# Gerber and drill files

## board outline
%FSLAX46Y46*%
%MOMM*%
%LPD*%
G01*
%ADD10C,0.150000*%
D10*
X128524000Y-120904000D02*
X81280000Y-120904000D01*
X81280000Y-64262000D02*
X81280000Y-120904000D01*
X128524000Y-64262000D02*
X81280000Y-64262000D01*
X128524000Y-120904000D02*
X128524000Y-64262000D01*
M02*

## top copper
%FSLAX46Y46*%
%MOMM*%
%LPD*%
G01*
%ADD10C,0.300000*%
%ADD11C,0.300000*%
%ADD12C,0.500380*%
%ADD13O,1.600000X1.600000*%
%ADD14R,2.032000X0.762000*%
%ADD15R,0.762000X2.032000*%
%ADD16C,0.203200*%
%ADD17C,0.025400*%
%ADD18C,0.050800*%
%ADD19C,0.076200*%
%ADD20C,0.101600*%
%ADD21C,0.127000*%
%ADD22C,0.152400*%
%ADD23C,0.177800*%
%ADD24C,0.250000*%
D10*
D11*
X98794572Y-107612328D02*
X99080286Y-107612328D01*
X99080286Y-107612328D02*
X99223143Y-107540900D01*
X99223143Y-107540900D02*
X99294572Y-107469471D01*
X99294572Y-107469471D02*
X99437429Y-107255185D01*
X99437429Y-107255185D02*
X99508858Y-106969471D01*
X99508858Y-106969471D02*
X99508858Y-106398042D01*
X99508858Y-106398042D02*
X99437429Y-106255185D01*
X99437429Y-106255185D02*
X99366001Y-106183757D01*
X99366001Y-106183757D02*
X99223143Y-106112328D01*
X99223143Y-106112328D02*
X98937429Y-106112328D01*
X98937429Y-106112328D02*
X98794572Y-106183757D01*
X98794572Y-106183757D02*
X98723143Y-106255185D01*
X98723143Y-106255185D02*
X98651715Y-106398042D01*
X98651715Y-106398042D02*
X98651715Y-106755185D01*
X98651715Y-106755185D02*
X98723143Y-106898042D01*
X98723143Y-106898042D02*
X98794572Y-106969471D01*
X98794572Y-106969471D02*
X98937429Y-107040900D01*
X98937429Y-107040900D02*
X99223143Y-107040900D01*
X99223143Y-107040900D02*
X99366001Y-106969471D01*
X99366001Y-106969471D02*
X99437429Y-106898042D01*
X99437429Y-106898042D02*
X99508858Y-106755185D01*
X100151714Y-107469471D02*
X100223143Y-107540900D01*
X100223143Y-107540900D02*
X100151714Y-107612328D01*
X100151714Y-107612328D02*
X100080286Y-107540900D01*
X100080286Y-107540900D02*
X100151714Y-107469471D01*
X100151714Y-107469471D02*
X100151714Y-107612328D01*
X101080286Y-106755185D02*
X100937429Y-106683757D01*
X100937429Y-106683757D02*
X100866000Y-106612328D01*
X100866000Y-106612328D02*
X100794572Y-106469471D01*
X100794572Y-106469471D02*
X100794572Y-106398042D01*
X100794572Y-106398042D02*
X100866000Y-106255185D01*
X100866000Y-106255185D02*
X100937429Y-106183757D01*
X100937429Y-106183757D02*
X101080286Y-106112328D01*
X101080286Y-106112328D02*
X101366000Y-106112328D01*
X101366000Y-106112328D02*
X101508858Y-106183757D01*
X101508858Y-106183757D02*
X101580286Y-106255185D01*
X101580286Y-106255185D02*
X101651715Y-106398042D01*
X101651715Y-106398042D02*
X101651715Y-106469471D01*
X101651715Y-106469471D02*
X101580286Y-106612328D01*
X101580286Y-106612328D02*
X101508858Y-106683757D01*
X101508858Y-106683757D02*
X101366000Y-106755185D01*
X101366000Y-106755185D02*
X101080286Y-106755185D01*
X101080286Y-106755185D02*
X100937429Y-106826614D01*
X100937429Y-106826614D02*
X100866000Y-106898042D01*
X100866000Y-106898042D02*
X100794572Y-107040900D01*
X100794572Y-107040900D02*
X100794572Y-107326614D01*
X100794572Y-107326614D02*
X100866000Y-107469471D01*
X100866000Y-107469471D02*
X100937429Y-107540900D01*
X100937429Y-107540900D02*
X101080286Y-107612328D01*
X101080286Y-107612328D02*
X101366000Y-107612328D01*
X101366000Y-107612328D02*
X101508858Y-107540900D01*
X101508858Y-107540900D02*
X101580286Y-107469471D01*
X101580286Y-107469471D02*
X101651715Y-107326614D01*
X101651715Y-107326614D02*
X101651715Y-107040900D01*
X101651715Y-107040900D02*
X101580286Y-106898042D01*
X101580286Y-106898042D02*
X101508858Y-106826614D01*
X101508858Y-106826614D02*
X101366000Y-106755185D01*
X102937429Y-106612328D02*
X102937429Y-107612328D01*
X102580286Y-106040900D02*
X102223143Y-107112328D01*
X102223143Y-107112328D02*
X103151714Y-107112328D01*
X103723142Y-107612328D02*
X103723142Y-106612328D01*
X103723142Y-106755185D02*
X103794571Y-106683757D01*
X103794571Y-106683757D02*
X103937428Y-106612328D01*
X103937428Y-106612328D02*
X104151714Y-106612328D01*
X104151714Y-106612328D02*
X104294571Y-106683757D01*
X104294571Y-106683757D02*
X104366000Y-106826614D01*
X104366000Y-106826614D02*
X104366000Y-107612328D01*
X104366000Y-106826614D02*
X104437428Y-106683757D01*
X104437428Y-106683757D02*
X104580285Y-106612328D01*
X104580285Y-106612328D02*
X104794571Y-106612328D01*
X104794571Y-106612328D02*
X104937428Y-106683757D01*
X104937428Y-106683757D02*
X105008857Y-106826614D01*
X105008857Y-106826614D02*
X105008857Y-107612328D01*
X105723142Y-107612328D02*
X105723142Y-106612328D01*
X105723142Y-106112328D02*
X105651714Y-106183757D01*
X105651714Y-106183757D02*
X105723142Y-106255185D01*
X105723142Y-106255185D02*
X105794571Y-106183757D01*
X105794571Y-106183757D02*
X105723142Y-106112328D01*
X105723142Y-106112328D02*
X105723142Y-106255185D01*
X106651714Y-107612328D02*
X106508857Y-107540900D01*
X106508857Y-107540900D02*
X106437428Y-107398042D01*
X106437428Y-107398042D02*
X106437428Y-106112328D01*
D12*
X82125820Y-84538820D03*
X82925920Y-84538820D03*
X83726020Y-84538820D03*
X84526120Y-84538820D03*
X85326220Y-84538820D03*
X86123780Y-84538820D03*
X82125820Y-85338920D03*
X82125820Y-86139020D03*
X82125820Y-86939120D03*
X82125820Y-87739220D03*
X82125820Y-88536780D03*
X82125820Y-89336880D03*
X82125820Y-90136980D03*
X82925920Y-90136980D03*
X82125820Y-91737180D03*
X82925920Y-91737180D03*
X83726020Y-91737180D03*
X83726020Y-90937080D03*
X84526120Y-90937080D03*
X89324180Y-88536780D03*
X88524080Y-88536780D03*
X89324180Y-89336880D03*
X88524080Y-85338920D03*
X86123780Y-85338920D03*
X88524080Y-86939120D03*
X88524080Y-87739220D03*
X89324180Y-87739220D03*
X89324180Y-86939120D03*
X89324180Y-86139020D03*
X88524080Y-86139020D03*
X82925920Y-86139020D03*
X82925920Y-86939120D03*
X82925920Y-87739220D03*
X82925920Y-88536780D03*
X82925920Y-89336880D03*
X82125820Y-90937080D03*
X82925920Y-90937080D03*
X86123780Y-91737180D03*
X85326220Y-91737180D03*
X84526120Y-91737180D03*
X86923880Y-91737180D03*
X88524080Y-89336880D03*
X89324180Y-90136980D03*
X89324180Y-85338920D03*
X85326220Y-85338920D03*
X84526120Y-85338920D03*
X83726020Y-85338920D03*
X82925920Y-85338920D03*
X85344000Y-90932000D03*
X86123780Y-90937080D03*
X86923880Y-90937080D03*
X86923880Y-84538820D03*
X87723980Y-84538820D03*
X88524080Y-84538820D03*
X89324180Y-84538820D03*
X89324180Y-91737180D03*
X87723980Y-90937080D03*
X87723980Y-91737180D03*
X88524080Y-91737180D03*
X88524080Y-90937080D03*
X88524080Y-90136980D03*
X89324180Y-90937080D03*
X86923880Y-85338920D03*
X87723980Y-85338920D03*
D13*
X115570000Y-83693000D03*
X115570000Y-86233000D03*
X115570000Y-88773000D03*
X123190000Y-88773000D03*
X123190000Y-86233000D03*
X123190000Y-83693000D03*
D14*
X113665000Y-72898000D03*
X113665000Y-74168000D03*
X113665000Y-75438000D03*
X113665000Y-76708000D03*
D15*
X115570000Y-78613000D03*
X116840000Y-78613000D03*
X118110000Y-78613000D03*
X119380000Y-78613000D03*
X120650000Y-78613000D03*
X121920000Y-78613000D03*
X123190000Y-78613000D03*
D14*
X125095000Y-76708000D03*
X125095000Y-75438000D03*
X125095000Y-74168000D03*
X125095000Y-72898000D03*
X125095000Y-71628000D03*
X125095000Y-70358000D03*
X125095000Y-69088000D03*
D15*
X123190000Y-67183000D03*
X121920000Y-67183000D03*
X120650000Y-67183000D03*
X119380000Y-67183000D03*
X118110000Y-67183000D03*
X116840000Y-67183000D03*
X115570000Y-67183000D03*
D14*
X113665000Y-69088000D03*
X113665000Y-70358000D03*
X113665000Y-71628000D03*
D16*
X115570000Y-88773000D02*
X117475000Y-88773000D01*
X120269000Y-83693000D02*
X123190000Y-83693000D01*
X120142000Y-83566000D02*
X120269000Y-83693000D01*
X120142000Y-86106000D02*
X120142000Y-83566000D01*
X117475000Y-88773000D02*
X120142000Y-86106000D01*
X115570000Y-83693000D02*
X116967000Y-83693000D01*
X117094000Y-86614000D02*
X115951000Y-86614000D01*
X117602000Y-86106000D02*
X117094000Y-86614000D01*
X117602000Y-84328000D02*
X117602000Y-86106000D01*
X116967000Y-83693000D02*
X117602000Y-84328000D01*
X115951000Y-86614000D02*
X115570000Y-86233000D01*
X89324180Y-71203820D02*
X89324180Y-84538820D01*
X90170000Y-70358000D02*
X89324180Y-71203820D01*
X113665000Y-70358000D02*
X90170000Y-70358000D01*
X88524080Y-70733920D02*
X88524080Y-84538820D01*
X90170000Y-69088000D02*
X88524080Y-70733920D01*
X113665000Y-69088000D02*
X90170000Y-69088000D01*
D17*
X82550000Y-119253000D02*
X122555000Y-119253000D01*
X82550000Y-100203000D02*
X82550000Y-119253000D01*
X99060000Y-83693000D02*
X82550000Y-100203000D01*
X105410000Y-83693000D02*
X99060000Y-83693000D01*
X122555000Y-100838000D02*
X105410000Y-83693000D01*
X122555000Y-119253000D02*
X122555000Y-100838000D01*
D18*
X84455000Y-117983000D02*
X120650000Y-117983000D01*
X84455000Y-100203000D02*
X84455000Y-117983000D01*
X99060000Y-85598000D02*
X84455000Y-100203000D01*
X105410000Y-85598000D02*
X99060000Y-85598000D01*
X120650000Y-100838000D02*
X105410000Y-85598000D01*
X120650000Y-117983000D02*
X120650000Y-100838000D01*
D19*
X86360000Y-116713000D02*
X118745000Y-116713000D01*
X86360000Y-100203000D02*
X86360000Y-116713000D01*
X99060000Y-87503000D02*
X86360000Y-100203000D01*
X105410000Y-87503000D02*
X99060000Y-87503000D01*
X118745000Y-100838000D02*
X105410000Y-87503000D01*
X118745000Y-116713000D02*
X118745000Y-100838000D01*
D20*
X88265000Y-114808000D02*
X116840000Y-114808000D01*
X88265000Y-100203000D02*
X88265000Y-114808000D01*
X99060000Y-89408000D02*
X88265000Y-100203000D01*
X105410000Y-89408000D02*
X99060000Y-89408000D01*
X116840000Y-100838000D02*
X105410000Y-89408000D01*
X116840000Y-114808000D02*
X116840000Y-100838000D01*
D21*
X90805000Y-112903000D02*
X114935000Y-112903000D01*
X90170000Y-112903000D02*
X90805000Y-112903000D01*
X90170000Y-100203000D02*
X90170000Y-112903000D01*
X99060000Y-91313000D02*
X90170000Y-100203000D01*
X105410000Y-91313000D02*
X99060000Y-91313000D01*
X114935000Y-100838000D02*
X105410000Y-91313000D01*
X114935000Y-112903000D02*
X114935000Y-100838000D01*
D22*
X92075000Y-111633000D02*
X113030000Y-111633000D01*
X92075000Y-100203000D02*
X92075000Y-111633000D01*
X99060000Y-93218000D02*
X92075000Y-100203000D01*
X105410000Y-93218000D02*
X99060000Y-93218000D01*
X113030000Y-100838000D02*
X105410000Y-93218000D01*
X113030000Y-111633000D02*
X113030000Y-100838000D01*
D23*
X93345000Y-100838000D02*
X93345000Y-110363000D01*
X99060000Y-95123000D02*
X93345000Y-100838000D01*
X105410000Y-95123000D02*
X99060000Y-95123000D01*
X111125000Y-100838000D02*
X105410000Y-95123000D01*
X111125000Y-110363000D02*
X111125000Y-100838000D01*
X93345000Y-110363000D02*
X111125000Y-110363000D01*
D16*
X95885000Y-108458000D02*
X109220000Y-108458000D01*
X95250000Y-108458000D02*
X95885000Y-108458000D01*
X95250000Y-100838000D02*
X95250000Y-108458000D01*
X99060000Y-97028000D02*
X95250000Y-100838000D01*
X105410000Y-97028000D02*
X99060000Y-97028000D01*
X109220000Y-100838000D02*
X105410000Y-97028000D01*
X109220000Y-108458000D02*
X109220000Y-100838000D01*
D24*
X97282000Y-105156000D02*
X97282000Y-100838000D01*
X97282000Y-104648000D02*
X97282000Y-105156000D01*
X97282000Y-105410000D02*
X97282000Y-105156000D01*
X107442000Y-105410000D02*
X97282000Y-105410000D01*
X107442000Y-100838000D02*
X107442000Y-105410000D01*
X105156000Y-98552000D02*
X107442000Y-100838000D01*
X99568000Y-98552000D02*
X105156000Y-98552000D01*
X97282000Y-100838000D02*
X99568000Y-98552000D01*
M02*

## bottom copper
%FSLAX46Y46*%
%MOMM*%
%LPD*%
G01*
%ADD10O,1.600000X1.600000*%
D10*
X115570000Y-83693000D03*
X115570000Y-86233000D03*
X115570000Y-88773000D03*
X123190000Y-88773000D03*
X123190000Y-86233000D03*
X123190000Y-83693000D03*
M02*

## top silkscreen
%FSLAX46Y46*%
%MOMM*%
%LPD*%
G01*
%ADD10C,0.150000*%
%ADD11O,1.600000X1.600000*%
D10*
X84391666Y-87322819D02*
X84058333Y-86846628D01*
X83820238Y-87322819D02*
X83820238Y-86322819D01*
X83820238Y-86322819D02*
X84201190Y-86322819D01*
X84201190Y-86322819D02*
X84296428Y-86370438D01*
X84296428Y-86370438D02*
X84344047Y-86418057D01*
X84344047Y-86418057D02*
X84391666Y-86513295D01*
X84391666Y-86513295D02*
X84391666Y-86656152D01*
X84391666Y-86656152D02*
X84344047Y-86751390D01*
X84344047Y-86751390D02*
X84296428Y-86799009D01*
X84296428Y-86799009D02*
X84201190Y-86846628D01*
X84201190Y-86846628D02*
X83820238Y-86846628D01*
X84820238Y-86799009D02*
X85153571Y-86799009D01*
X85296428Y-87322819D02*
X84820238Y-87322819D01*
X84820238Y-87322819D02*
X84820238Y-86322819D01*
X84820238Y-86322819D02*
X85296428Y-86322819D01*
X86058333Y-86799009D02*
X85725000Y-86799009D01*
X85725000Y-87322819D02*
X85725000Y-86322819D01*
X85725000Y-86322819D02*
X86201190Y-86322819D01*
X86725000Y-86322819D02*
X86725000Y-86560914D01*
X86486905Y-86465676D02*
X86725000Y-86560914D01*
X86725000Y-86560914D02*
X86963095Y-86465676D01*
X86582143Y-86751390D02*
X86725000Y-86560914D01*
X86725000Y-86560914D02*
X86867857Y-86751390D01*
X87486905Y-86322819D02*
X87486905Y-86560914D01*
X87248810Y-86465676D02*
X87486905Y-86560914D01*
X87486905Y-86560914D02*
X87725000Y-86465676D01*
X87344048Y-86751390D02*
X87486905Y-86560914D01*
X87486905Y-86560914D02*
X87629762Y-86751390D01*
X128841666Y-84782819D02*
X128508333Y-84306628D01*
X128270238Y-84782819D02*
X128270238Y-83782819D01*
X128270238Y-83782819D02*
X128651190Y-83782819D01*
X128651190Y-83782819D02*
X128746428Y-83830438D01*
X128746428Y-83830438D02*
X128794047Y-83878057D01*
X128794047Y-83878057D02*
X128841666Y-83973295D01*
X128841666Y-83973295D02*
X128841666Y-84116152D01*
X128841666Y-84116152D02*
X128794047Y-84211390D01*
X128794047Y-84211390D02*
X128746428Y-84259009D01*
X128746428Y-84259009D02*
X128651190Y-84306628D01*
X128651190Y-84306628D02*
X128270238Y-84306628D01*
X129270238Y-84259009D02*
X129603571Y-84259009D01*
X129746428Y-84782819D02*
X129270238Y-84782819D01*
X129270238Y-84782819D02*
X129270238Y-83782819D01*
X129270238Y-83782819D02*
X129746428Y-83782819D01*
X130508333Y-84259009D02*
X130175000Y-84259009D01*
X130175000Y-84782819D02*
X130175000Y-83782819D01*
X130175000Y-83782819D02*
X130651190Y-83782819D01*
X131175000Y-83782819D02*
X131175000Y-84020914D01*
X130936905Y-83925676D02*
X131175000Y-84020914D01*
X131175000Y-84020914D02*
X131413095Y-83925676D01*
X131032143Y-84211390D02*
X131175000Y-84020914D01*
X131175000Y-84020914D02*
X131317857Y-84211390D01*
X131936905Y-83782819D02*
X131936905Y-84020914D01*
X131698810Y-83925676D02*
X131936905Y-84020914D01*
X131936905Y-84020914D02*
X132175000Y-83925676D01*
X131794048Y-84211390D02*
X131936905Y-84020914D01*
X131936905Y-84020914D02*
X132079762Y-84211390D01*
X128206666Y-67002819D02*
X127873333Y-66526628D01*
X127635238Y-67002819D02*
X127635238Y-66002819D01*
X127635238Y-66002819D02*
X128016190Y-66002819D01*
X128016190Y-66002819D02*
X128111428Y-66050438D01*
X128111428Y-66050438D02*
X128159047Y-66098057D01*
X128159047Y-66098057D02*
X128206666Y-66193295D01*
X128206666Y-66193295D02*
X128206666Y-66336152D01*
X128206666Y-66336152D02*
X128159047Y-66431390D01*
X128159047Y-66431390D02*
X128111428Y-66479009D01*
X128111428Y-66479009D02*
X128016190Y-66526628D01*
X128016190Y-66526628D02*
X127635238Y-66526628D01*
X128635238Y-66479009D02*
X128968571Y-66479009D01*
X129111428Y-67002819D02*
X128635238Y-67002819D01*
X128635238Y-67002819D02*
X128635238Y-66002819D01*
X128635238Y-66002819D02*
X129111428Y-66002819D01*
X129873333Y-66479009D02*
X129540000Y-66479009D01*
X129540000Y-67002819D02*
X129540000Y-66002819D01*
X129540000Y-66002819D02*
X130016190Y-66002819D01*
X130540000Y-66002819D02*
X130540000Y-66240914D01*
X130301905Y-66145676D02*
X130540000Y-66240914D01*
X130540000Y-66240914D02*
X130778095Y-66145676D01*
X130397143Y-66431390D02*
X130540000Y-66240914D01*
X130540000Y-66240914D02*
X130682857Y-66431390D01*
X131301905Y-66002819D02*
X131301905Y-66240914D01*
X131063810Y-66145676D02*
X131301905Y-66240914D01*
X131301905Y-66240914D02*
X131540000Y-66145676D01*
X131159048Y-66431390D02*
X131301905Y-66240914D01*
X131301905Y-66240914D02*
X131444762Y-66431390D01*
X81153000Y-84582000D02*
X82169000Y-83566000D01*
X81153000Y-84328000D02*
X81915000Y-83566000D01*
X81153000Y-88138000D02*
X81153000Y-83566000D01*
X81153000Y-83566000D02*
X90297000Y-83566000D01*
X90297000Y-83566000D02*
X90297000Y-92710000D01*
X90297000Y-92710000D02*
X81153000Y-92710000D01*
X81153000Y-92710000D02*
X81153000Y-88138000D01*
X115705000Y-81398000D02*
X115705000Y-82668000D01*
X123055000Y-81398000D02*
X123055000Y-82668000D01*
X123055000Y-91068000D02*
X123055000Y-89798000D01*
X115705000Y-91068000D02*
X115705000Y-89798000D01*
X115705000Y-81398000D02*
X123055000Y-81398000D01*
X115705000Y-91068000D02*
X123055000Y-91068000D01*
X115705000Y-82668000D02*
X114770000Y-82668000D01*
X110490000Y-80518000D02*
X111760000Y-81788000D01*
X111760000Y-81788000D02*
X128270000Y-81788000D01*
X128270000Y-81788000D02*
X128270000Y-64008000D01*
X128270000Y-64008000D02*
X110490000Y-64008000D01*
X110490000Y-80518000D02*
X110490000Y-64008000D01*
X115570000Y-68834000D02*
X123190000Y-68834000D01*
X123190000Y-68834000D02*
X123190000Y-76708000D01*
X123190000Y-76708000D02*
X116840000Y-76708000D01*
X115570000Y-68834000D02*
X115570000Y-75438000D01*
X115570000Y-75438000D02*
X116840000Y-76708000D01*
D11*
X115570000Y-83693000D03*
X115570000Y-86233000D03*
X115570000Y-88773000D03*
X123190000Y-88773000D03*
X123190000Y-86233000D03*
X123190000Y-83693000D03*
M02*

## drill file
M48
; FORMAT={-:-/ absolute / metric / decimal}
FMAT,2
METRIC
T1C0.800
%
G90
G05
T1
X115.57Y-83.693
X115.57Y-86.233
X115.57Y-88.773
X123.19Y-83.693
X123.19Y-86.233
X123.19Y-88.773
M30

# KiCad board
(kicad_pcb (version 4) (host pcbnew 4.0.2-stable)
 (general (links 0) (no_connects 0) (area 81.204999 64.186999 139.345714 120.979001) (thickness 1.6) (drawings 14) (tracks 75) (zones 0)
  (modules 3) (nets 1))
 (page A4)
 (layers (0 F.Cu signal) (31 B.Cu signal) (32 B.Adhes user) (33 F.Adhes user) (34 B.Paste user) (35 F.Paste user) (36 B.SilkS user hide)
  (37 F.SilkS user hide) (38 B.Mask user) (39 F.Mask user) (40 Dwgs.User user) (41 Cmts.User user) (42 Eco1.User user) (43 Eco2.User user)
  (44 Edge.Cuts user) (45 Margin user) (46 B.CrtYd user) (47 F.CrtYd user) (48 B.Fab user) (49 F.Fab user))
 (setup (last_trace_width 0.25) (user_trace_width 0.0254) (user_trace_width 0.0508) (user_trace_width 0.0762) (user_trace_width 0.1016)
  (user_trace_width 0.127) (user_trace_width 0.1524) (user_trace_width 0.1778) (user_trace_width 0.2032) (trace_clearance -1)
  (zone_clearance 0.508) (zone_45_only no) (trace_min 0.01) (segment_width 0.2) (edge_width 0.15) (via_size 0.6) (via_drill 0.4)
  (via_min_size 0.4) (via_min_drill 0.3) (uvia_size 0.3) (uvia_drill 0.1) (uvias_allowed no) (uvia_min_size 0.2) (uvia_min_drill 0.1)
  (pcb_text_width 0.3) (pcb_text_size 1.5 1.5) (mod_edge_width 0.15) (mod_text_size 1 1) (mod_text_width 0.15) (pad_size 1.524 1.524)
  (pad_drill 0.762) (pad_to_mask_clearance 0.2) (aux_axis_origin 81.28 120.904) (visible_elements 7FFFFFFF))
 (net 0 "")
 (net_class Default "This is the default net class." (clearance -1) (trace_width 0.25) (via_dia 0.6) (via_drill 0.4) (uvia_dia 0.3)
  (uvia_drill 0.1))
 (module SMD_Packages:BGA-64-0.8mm (layer F.Cu) (at 85.725 88.138)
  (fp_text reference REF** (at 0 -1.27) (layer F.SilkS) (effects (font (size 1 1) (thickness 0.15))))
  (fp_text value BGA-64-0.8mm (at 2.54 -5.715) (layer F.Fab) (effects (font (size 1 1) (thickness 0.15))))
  (fp_line (start -4.572 -3.556) (end -3.556 -4.572) (layer F.SilkS) (width 0.15))
  (fp_line (start -4.572 -3.81) (end -3.81 -4.572) (layer F.SilkS) (width 0.15))
  (fp_line (start -4.572 0) (end -4.572 -4.572) (layer F.SilkS) (width 0.15))
  (fp_line (start -4.572 -4.572) (end 4.572 -4.572) (layer F.SilkS) (width 0.15))
  (fp_line (start 4.572 -4.572) (end 4.572 4.572) (layer F.SilkS) (width 0.15))
  (fp_line (start 4.572 4.572) (end -4.572 4.572) (layer F.SilkS) (width 0.15))
  (fp_line (start -4.572 4.572) (end -4.572 0) (layer F.SilkS) (width 0.15))
  (pad A1 smd circle (at -3.59918 -3.59918) (size 0.50038 0.50038) (layers F.Cu F.Paste F.Mask))
  (pad A2 smd circle (at -2.79908 -3.59918) (size 0.50038 0.50038) (layers F.Cu F.Paste F.Mask))
  (pad A3 smd circle (at -1.99898 -3.59918) (size 0.50038 0.50038) (layers F.Cu F.Paste F.Mask))
  (pad A4 smd circle (at -1.19888 -3.59918) (size 0.50038 0.50038) (layers F.Cu F.Paste F.Mask))
  (pad A5 smd circle (at -0.39878 -3.59918) (size 0.50038 0.50038) (layers F.Cu F.Paste F.Mask))
  (pad A6 smd circle (at 0.39878 -3.59918) (size 0.50038 0.50038) (layers F.Cu F.Paste F.Mask))
  (pad B1 smd circle (at -3.59918 -2.79908) (size 0.50038 0.50038) (layers F.Cu F.Paste F.Mask))
  (pad C1 smd circle (at -3.59918 -1.99898) (size 0.50038 0.50038) (layers F.Cu F.Paste F.Mask))
  (pad D1 smd circle (at -3.59918 -1.19888) (size 0.50038 0.50038) (layers F.Cu F.Paste F.Mask))
  (pad E1 smd circle (at -3.59918 -0.39878) (size 0.50038 0.50038) (layers F.Cu F.Paste F.Mask))
  (pad F1 smd circle (at -3.59918 0.39878) (size 0.50038 0.50038) (layers F.Cu F.Paste F.Mask))
  (pad G1 smd circle (at -3.59918 1.19888) (size 0.50038 0.50038) (layers F.Cu F.Paste F.Mask))
  (pad H1 smd circle (at -3.59918 1.99898) (size 0.50038 0.50038) (layers F.Cu F.Paste F.Mask))
  (pad H2 smd circle (at -2.79908 1.99898) (size 0.50038 0.50038) (layers F.Cu F.Paste F.Mask))
  (pad K1 smd circle (at -3.59918 3.59918) (size 0.50038 0.50038) (layers F.Cu F.Paste F.Mask))
  (pad K2 smd circle (at -2.79908 3.59918) (size 0.50038 0.50038) (layers F.Cu F.Paste F.Mask))
  (pad K3 smd circle (at -1.99898 3.59918) (size 0.50038 0.50038) (layers F.Cu F.Paste F.Mask))
  (pad J3 smd circle (at -1.99898 2.79908) (size 0.50038 0.50038) (layers F.Cu F.Paste F.Mask))
  (pad J4 smd circle (at -1.19888 2.79908) (size 0.50038 0.50038) (layers F.Cu F.Paste F.Mask))
  (pad F10 smd circle (at 3.59918 0.39878) (size 0.50038 0.50038) (layers F.Cu F.Paste F.Mask))
  (pad F9 smd circle (at 2.79908 0.39878) (size 0.50038 0.50038) (layers F.Cu F.Paste F.Mask))
  (pad G10 smd circle (at 3.59918 1.19888) (size 0.50038 0.50038) (layers F.Cu F.Paste F.Mask))
  (pad B9 smd circle (at 2.79908 -2.79908) (size 0.50038 0.50038) (layers F.Cu F.Paste F.Mask))
  (pad B6 smd circle (at 0.39878 -2.79908) (size 0.50038 0.50038) (layers F.Cu F.Paste F.Mask))
  (pad D9 smd circle (at 2.79908 -1.19888) (size 0.50038 0.50038) (layers F.Cu F.Paste F.Mask))
  (pad E9 smd circle (at 2.79908 -0.39878) (size 0.50038 0.50038) (layers F.Cu F.Paste F.Mask))
  (pad E10 smd circle (at 3.59918 -0.39878) (size 0.50038 0.50038) (layers F.Cu F.Paste F.Mask))
  (pad D10 smd circle (at 3.59918 -1.19888) (size 0.50038 0.50038) (layers F.Cu F.Paste F.Mask))
  (pad C10 smd circle (at 3.59918 -1.99898) (size 0.50038 0.50038) (layers F.Cu F.Paste F.Mask))
  (pad C9 smd circle (at 2.79908 -1.99898) (size 0.50038 0.50038) (layers F.Cu F.Paste F.Mask))
  (pad C2 smd circle (at -2.79908 -1.99898) (size 0.50038 0.50038) (layers F.Cu F.Paste F.Mask))
  (pad D2 smd circle (at -2.79908 -1.19888) (size 0.50038 0.50038) (layers F.Cu F.Paste F.Mask))
  (pad E2 smd circle (at -2.79908 -0.39878) (size 0.50038 0.50038) (layers F.Cu F.Paste F.Mask))
  (pad F2 smd circle (at -2.79908 0.39878) (size 0.50038 0.50038) (layers F.Cu F.Paste F.Mask))
  (pad G2 smd circle (at -2.79908 1.19888) (size 0.50038 0.50038) (layers F.Cu F.Paste F.Mask))
  (pad J1 smd circle (at -3.59918 2.79908) (size 0.50038 0.50038) (layers F.Cu F.Paste F.Mask))
  (pad J2 smd circle (at -2.79908 2.79908) (size 0.50038 0.50038) (layers F.Cu F.Paste F.Mask))
  (pad K6 smd circle (at 0.39878 3.59918) (size 0.50038 0.50038) (layers F.Cu F.Paste F.Mask))
  (pad K5 smd circle (at -0.39878 3.59918) (size 0.50038 0.50038) (layers F.Cu F.Paste F.Mask))
  (pad K4 smd circle (at -1.19888 3.59918) (size 0.50038 0.50038) (layers F.Cu F.Paste F.Mask))
  (pad K7 smd circle (at 1.19888 3.59918) (size 0.50038 0.50038) (layers F.Cu F.Paste F.Mask))
  (pad G9 smd circle (at 2.79908 1.19888) (size 0.50038 0.50038) (layers F.Cu F.Paste F.Mask))
  (pad H10 smd circle (at 3.59918 1.99898) (size 0.50038 0.50038) (layers F.Cu F.Paste F.Mask))
  (pad B10 smd circle (at 3.59918 -2.79908) (size 0.50038 0.50038) (layers F.Cu F.Paste F.Mask))
  (pad B5 smd circle (at -0.39878 -2.79908) (size 0.50038 0.50038) (layers F.Cu F.Paste F.Mask))
  (pad B4 smd circle (at -1.19888 -2.79908) (size 0.50038 0.50038) (layers F.Cu F.Paste F.Mask))
  (pad B3 smd circle (at -1.99898 -2.79908) (size 0.50038 0.50038) (layers F.Cu F.Paste F.Mask))
  (pad B2 smd circle (at -2.79908 -2.79908) (size 0.50038 0.50038) (layers F.Cu F.Paste F.Mask))
  (pad J5 smd circle (at -0.381 2.794) (size 0.50038 0.50038) (layers F.Cu F.Paste F.Mask))
  (pad J6 smd circle (at 0.39878 2.79908) (size 0.50038 0.50038) (layers F.Cu F.Paste F.Mask))
  (pad J7 smd circle (at 1.19888 2.79908) (size 0.50038 0.50038) (layers F.Cu F.Paste F.Mask))
  (pad A7 smd circle (at 1.19888 -3.59918) (size 0.50038 0.50038) (layers F.Cu F.Paste F.Mask))
  (pad A8 smd circle (at 1.99898 -3.59918) (size 0.50038 0.50038) (layers F.Cu F.Paste F.Mask))
  (pad A9 smd circle (at 2.79908 -3.59918) (size 0.50038 0.50038) (layers F.Cu F.Paste F.Mask))
  (pad A10 smd circle (at 3.59918 -3.59918) (size 0.50038 0.50038) (layers F.Cu F.Paste F.Mask))
  (pad K10 smd circle (at 3.59918 3.59918) (size 0.50038 0.50038) (layers F.Cu F.Paste F.Mask))
  (pad J8 smd circle (at 1.99898 2.79908) (size 0.50038 0.50038) (layers F.Cu F.Paste F.Mask))
  (pad K8 smd circle (at 1.99898 3.59918) (size 0.50038 0.50038) (layers F.Cu F.Paste F.Mask))
  (pad K9 smd circle (at 2.79908 3.59918) (size 0.50038 0.50038) (layers F.Cu F.Paste F.Mask))
  (pad J9 smd circle (at 2.79908 2.79908) (size 0.50038 0.50038) (layers F.Cu F.Paste F.Mask))
  (pad H9 smd circle (at 2.79908 1.99898) (size 0.50038 0.50038) (layers F.Cu F.Paste F.Mask))
  (pad J10 smd circle (at 3.59918 2.79908) (size 0.50038 0.50038) (layers F.Cu F.Paste F.Mask))
  (pad B7 smd circle (at 1.19888 -2.79908) (size 0.50038 0.50038) (layers F.Cu F.Paste F.Mask))
  (pad B8 smd circle (at 1.99898 -2.79908) (size 0.50038 0.50038) (layers F.Cu F.Paste F.Mask)))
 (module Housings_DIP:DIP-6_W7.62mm (layer F.Cu) (at 115.57 83.693)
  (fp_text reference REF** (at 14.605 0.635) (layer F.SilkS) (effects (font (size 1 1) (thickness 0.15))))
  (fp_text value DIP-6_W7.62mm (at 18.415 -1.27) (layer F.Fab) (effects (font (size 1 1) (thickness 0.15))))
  (fp_line (start 0.135 -2.295) (end 0.135 -1.025) (layer F.SilkS) (width 0.15))
  (fp_line (start 7.485 -2.295) (end 7.485 -1.025) (layer F.SilkS) (width 0.15))
  (fp_line (start 7.485 7.375) (end 7.485 6.105) (layer F.SilkS) (width 0.15))
  (fp_line (start 0.135 7.375) (end 0.135 6.105) (layer F.SilkS) (width 0.15))
  (fp_line (start 0.135 -2.295) (end 7.485 -2.295) (layer F.SilkS) (width 0.15))
  (fp_line (start 0.135 7.375) (end 7.485 7.375) (layer F.SilkS) (width 0.15))
  (fp_line (start 0.135 -1.025) (end -0.8 -1.025) (layer F.SilkS) (width 0.15))
  (pad 1 thru_hole oval (at 0 0) (size 1.6 1.6) (drill 0.8) (layers *.Cu *.Mask F.SilkS))
  (pad 2 thru_hole oval (at 0 2.54) (size 1.6 1.6) (drill 0.8) (layers *.Cu *.Mask F.SilkS))
  (pad 3 thru_hole oval (at 0 5.08) (size 1.6 1.6) (drill 0.8) (layers *.Cu *.Mask F.SilkS))
  (pad 4 thru_hole oval (at 7.62 5.08) (size 1.6 1.6) (drill 0.8) (layers *.Cu *.Mask F.SilkS))
  (pad 5 thru_hole oval (at 7.62 2.54) (size 1.6 1.6) (drill 0.8) (layers *.Cu *.Mask F.SilkS))
  (pad 6 thru_hole oval (at 7.62 0) (size 1.6 1.6) (drill 0.8) (layers *.Cu *.Mask F.SilkS)))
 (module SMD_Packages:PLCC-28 (layer F.Cu) (at 119.38 72.898)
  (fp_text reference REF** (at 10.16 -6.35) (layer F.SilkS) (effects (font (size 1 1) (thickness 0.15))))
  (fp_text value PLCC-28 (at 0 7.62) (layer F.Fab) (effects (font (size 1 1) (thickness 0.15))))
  (fp_line (start -8.89 7.62) (end -7.62 8.89) (layer F.SilkS) (width 0.15))
  (fp_line (start -7.62 8.89) (end 8.89 8.89) (layer F.SilkS) (width 0.15))
  (fp_line (start 8.89 8.89) (end 8.89 -8.89) (layer F.SilkS) (width 0.15))
  (fp_line (start 8.89 -8.89) (end -8.89 -8.89) (layer F.SilkS) (width 0.15))
  (fp_line (start -8.89 7.62) (end -8.89 -8.89) (layer F.SilkS) (width 0.15))
  (fp_line (start -3.81 -4.064) (end 3.81 -4.064) (layer F.SilkS) (width 0.15))
  (fp_line (start 3.81 -4.064) (end 3.81 3.81) (layer F.SilkS) (width 0.15))
  (fp_line (start 3.81 3.81) (end -2.54 3.81) (layer F.SilkS) (width 0.15))
  (fp_line (start -3.81 -4.064) (end -3.81 2.54) (layer F.SilkS) (width 0.15))
  (fp_line (start -3.81 2.54) (end -2.54 3.81) (layer F.SilkS) (width 0.15))
  (pad 1 smd rect (at -5.715 0) (size 2.032 0.762) (layers F.Cu F.Paste F.Mask))
  (pad 2 smd rect (at -5.715 1.27) (size 2.032 0.762) (layers F.Cu F.Paste F.Mask))
  (pad 3 smd rect (at -5.715 2.54) (size 2.032 0.762) (layers F.Cu F.Paste F.Mask))
  (pad 4 smd rect (at -5.715 3.81) (size 2.032 0.762) (layers F.Cu F.Paste F.Mask))
  (pad 5 smd rect (at -3.81 5.715) (size 0.762 2.032) (layers F.Cu F.Paste F.Mask))
  (pad 6 smd rect (at -2.54 5.715) (size 0.762 2.032) (layers F.Cu F.Paste F.Mask))
  (pad 7 smd rect (at -1.27 5.715) (size 0.762 2.032) (layers F.Cu F.Paste F.Mask))
  (pad 8 smd rect (at 0 5.715) (size 0.762 2.032) (layers F.Cu F.Paste F.Mask))
  (pad 9 smd rect (at 1.27 5.715) (size 0.762 2.032) (layers F.Cu F.Paste F.Mask))
  (pad 10 smd rect (at 2.54 5.715) (size 0.762 2.032) (layers F.Cu F.Paste F.Mask))
  (pad 11 smd rect (at 3.81 5.715) (size 0.762 2.032) (layers F.Cu F.Paste F.Mask))
  (pad 12 smd rect (at 5.715 3.81) (size 2.032 0.762) (layers F.Cu F.Paste F.Mask))
  (pad 13 smd rect (at 5.715 2.54) (size 2.032 0.762) (layers F.Cu F.Paste F.Mask))
  (pad 14 smd rect (at 5.715 1.27) (size 2.032 0.762) (layers F.Cu F.Paste F.Mask))
  (pad 15 smd rect (at 5.715 0) (size 2.032 0.762) (layers F.Cu F.Paste F.Mask))
  (pad 16 smd rect (at 5.715 -1.27) (size 2.032 0.762) (layers F.Cu F.Paste F.Mask))
  (pad 17 smd rect (at 5.715 -2.54) (size 2.032 0.762) (layers F.Cu F.Paste F.Mask))
  (pad 18 smd rect (at 5.715 -3.81) (size 2.032 0.762) (layers F.Cu F.Paste F.Mask))
  (pad 19 smd rect (at 3.81 -5.715) (size 0.762 2.032) (layers F.Cu F.Paste F.Mask))
  (pad 20 smd rect (at 2.54 -5.715) (size 0.762 2.032) (layers F.Cu F.Paste F.Mask))
  (pad 21 smd rect (at 1.27 -5.715) (size 0.762 2.032) (layers F.Cu F.Paste F.Mask))
  (pad 22 smd rect (at 0 -5.715) (size 0.762 2.032) (layers F.Cu F.Paste F.Mask))
  (pad 23 smd rect (at -1.27 -5.715) (size 0.762 2.032) (layers F.Cu F.Paste F.Mask))
  (pad 24 smd rect (at -2.54 -5.715) (size 0.762 2.032) (layers F.Cu F.Paste F.Mask))
  (pad 25 smd rect (at -3.81 -5.715) (size 0.762 2.032) (layers F.Cu F.Paste F.Mask))
  (pad 26 smd rect (at -5.715 -3.81) (size 2.032 0.762) (layers F.Cu F.Paste F.Mask))
  (pad 27 smd rect (at -5.715 -2.54) (size 2.032 0.762) (layers F.Cu F.Paste F.Mask))
  (pad 28 smd rect (at -5.715 -1.27) (size 2.032 0.762) (layers F.Cu F.Paste F.Mask)))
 (gr_line (start 128.524 120.904) (end 81.28 120.904) (angle 90) (layer Edge.Cuts) (width 0.15))
 (gr_line (start 81.28 64.262) (end 81.28 120.904) (angle 90) (layer Edge.Cuts) (width 0.15))
 (gr_line (start 128.524 64.262) (end 81.28 64.262) (angle 90) (layer Edge.Cuts) (width 0.15))
 (gr_line (start 128.524 120.904) (end 128.524 64.262) (angle 90) (layer Edge.Cuts) (width 0.15))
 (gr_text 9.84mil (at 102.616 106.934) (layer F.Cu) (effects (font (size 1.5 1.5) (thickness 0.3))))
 (segment (start 115.57 88.773) (end 117.475 88.773) (width 0.2032) (layer F.Cu) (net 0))
 (segment (start 120.269 83.693) (end 123.19 83.693) (width 0.2032) (layer F.Cu) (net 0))
 (segment (start 120.142 83.566) (end 120.269 83.693) (width 0.2032) (layer F.Cu) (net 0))
 (segment (start 120.142 86.106) (end 120.142 83.566) (width 0.2032) (layer F.Cu) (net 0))
 (segment (start 117.475 88.773) (end 120.142 86.106) (width 0.2032) (layer F.Cu) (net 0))
 (segment (start 115.57 83.693) (end 116.967 83.693) (width 0.2032) (layer F.Cu) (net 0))
 (segment (start 117.094 86.614) (end 115.951 86.614) (width 0.2032) (layer F.Cu) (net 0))
 (segment (start 117.602 86.106) (end 117.094 86.614) (width 0.2032) (layer F.Cu) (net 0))
 (segment (start 117.602 84.328) (end 117.602 86.106) (width 0.2032) (layer F.Cu) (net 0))
 (segment (start 116.967 83.693) (end 117.602 84.328) (width 0.2032) (layer F.Cu) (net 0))
 (segment (start 115.951 86.614) (end 115.57 86.233) (width 0.2032) (layer F.Cu) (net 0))
 (segment (start 89.32418 71.20382) (end 89.32418 84.53882) (width 0.2032) (layer F.Cu) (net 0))
 (segment (start 90.17 70.358) (end 89.32418 71.20382) (width 0.2032) (layer F.Cu) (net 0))
 (segment (start 113.665 70.358) (end 90.17 70.358) (width 0.2032) (layer F.Cu) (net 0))
 (segment (start 88.52408 70.73392) (end 88.52408 84.53882) (width 0.2032) (layer F.Cu) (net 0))
 (segment (start 90.17 69.088) (end 88.52408 70.73392) (width 0.2032) (layer F.Cu) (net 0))
 (segment (start 113.665 69.088) (end 90.17 69.088) (width 0.2032) (layer F.Cu) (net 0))
 (segment (start 82.55 119.253) (end 122.555 119.253) (width 0.0254) (layer F.Cu) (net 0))
 (segment (start 82.55 100.203) (end 82.55 119.253) (width 0.0254) (layer F.Cu) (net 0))
 (segment (start 99.06 83.693) (end 82.55 100.203) (width 0.0254) (layer F.Cu) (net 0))
 (segment (start 105.41 83.693) (end 99.06 83.693) (width 0.0254) (layer F.Cu) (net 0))
 (segment (start 122.555 100.838) (end 105.41 83.693) (width 0.0254) (layer F.Cu) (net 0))
 (segment (start 122.555 119.253) (end 122.555 100.838) (width 0.0254) (layer F.Cu) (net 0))
 (segment (start 84.455 117.983) (end 120.65 117.983) (width 0.0508) (layer F.Cu) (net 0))
 (segment (start 84.455 100.203) (end 84.455 117.983) (width 0.0508) (layer F.Cu) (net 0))
 (segment (start 99.06 85.598) (end 84.455 100.203) (width 0.0508) (layer F.Cu) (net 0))
 (segment (start 105.41 85.598) (end 99.06 85.598) (width 0.0508) (layer F.Cu) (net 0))
 (segment (start 120.65 100.838) (end 105.41 85.598) (width 0.0508) (layer F.Cu) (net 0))
 (segment (start 120.65 117.983) (end 120.65 100.838) (width 0.0508) (layer F.Cu) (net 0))
 (segment (start 86.36 116.713) (end 118.745 116.713) (width 0.0762) (layer F.Cu) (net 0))
 (segment (start 86.36 100.203) (end 86.36 116.713) (width 0.0762) (layer F.Cu) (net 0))
 (segment (start 99.06 87.503) (end 86.36 100.203) (width 0.0762) (layer F.Cu) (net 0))
 (segment (start 105.41 87.503) (end 99.06 87.503) (width 0.0762) (layer F.Cu) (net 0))
 (segment (start 118.745 100.838) (end 105.41 87.503) (width 0.0762) (layer F.Cu) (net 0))
 (segment (start 118.745 116.713) (end 118.745 100.838) (width 0.0762) (layer F.Cu) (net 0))
 (segment (start 88.265 114.808) (end 116.84 114.808) (width 0.1016) (layer F.Cu) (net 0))
 (segment (start 88.265 100.203) (end 88.265 114.808) (width 0.1016) (layer F.Cu) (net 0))
 (segment (start 99.06 89.408) (end 88.265 100.203) (width 0.1016) (layer F.Cu) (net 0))
 (segment (start 105.41 89.408) (end 99.06 89.408) (width 0.1016) (layer F.Cu) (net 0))
 (segment (start 116.84 100.838) (end 105.41 89.408) (width 0.1016) (layer F.Cu) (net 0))
 (segment (start 116.84 114.808) (end 116.84 100.838) (width 0.1016) (layer F.Cu) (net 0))
 (segment (start 90.805 112.903) (end 114.935 112.903) (width 0.127) (layer F.Cu) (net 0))
 (segment (start 90.17 112.903) (end 90.805 112.903) (width 0.127) (layer F.Cu) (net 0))
 (segment (start 90.17 100.203) (end 90.17 112.903) (width 0.127) (layer F.Cu) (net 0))
 (segment (start 99.06 91.313) (end 90.17 100.203) (width 0.127) (layer F.Cu) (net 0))
 (segment (start 105.41 91.313) (end 99.06 91.313) (width 0.127) (layer F.Cu) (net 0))
 (segment (start 114.935 100.838) (end 105.41 91.313) (width 0.127) (layer F.Cu) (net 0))
 (segment (start 114.935 112.903) (end 114.935 100.838) (width 0.127) (layer F.Cu) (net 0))
 (segment (start 92.075 111.633) (end 113.03 111.633) (width 0.1524) (layer F.Cu) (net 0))
 (segment (start 92.075 100.203) (end 92.075 111.633) (width 0.1524) (layer F.Cu) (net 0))
 (segment (start 99.06 93.218) (end 92.075 100.203) (width 0.1524) (layer F.Cu) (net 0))
 (segment (start 105.41 93.218) (end 99.06 93.218) (width 0.1524) (layer F.Cu) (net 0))
 (segment (start 113.03 100.838) (end 105.41 93.218) (width 0.1524) (layer F.Cu) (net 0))
 (segment (start 113.03 111.633) (end 113.03 100.838) (width 0.1524) (layer F.Cu) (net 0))
 (segment (start 93.345 100.838) (end 93.345 110.363) (width 0.1778) (layer F.Cu) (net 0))
 (segment (start 99.06 95.123) (end 93.345 100.838) (width 0.1778) (layer F.Cu) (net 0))
 (segment (start 105.41 95.123) (end 99.06 95.123) (width 0.1778) (layer F.Cu) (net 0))
 (segment (start 111.125 100.838) (end 105.41 95.123) (width 0.1778) (layer F.Cu) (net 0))
 (segment (start 111.125 110.363) (end 111.125 100.838) (width 0.1778) (layer F.Cu) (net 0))
 (segment (start 93.345 110.363) (end 111.125 110.363) (width 0.1778) (layer F.Cu) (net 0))
 (segment (start 95.885 108.458) (end 109.22 108.458) (width 0.2032) (layer F.Cu) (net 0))
 (segment (start 95.25 108.458) (end 95.885 108.458) (width 0.2032) (layer F.Cu) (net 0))
 (segment (start 95.25 100.838) (end 95.25 108.458) (width 0.2032) (layer F.Cu) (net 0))
 (segment (start 99.06 97.028) (end 95.25 100.838) (width 0.2032) (layer F.Cu) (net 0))
 (segment (start 105.41 97.028) (end 99.06 97.028) (width 0.2032) (layer F.Cu) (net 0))
 (segment (start 109.22 100.838) (end 105.41 97.028) (width 0.2032) (layer F.Cu) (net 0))
 (segment (start 109.22 108.458) (end 109.22 100.838) (width 0.2032) (layer F.Cu) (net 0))
 (segment (start 97.282 105.156) (end 97.282 100.838) (width 0.25) (layer F.Cu) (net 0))
 (segment (start 97.282 104.648) (end 97.282 105.156) (width 0.25) (layer F.Cu) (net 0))
 (segment (start 97.282 105.41) (end 97.282 105.156) (width 0.25) (layer F.Cu) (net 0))
 (segment (start 107.442 105.41) (end 97.282 105.41) (width 0.25) (layer F.Cu) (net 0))
 (segment (start 107.442 100.838) (end 107.442 105.41) (width 0.25) (layer F.Cu) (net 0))
 (segment (start 105.156 98.552) (end 107.442 100.838) (width 0.25) (layer F.Cu) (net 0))
 (segment (start 99.568 98.552) (end 105.156 98.552) (width 0.25) (layer F.Cu) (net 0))
 (segment (start 97.282 100.838) (end 99.568 98.552) (width 0.25) (layer F.Cu) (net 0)))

